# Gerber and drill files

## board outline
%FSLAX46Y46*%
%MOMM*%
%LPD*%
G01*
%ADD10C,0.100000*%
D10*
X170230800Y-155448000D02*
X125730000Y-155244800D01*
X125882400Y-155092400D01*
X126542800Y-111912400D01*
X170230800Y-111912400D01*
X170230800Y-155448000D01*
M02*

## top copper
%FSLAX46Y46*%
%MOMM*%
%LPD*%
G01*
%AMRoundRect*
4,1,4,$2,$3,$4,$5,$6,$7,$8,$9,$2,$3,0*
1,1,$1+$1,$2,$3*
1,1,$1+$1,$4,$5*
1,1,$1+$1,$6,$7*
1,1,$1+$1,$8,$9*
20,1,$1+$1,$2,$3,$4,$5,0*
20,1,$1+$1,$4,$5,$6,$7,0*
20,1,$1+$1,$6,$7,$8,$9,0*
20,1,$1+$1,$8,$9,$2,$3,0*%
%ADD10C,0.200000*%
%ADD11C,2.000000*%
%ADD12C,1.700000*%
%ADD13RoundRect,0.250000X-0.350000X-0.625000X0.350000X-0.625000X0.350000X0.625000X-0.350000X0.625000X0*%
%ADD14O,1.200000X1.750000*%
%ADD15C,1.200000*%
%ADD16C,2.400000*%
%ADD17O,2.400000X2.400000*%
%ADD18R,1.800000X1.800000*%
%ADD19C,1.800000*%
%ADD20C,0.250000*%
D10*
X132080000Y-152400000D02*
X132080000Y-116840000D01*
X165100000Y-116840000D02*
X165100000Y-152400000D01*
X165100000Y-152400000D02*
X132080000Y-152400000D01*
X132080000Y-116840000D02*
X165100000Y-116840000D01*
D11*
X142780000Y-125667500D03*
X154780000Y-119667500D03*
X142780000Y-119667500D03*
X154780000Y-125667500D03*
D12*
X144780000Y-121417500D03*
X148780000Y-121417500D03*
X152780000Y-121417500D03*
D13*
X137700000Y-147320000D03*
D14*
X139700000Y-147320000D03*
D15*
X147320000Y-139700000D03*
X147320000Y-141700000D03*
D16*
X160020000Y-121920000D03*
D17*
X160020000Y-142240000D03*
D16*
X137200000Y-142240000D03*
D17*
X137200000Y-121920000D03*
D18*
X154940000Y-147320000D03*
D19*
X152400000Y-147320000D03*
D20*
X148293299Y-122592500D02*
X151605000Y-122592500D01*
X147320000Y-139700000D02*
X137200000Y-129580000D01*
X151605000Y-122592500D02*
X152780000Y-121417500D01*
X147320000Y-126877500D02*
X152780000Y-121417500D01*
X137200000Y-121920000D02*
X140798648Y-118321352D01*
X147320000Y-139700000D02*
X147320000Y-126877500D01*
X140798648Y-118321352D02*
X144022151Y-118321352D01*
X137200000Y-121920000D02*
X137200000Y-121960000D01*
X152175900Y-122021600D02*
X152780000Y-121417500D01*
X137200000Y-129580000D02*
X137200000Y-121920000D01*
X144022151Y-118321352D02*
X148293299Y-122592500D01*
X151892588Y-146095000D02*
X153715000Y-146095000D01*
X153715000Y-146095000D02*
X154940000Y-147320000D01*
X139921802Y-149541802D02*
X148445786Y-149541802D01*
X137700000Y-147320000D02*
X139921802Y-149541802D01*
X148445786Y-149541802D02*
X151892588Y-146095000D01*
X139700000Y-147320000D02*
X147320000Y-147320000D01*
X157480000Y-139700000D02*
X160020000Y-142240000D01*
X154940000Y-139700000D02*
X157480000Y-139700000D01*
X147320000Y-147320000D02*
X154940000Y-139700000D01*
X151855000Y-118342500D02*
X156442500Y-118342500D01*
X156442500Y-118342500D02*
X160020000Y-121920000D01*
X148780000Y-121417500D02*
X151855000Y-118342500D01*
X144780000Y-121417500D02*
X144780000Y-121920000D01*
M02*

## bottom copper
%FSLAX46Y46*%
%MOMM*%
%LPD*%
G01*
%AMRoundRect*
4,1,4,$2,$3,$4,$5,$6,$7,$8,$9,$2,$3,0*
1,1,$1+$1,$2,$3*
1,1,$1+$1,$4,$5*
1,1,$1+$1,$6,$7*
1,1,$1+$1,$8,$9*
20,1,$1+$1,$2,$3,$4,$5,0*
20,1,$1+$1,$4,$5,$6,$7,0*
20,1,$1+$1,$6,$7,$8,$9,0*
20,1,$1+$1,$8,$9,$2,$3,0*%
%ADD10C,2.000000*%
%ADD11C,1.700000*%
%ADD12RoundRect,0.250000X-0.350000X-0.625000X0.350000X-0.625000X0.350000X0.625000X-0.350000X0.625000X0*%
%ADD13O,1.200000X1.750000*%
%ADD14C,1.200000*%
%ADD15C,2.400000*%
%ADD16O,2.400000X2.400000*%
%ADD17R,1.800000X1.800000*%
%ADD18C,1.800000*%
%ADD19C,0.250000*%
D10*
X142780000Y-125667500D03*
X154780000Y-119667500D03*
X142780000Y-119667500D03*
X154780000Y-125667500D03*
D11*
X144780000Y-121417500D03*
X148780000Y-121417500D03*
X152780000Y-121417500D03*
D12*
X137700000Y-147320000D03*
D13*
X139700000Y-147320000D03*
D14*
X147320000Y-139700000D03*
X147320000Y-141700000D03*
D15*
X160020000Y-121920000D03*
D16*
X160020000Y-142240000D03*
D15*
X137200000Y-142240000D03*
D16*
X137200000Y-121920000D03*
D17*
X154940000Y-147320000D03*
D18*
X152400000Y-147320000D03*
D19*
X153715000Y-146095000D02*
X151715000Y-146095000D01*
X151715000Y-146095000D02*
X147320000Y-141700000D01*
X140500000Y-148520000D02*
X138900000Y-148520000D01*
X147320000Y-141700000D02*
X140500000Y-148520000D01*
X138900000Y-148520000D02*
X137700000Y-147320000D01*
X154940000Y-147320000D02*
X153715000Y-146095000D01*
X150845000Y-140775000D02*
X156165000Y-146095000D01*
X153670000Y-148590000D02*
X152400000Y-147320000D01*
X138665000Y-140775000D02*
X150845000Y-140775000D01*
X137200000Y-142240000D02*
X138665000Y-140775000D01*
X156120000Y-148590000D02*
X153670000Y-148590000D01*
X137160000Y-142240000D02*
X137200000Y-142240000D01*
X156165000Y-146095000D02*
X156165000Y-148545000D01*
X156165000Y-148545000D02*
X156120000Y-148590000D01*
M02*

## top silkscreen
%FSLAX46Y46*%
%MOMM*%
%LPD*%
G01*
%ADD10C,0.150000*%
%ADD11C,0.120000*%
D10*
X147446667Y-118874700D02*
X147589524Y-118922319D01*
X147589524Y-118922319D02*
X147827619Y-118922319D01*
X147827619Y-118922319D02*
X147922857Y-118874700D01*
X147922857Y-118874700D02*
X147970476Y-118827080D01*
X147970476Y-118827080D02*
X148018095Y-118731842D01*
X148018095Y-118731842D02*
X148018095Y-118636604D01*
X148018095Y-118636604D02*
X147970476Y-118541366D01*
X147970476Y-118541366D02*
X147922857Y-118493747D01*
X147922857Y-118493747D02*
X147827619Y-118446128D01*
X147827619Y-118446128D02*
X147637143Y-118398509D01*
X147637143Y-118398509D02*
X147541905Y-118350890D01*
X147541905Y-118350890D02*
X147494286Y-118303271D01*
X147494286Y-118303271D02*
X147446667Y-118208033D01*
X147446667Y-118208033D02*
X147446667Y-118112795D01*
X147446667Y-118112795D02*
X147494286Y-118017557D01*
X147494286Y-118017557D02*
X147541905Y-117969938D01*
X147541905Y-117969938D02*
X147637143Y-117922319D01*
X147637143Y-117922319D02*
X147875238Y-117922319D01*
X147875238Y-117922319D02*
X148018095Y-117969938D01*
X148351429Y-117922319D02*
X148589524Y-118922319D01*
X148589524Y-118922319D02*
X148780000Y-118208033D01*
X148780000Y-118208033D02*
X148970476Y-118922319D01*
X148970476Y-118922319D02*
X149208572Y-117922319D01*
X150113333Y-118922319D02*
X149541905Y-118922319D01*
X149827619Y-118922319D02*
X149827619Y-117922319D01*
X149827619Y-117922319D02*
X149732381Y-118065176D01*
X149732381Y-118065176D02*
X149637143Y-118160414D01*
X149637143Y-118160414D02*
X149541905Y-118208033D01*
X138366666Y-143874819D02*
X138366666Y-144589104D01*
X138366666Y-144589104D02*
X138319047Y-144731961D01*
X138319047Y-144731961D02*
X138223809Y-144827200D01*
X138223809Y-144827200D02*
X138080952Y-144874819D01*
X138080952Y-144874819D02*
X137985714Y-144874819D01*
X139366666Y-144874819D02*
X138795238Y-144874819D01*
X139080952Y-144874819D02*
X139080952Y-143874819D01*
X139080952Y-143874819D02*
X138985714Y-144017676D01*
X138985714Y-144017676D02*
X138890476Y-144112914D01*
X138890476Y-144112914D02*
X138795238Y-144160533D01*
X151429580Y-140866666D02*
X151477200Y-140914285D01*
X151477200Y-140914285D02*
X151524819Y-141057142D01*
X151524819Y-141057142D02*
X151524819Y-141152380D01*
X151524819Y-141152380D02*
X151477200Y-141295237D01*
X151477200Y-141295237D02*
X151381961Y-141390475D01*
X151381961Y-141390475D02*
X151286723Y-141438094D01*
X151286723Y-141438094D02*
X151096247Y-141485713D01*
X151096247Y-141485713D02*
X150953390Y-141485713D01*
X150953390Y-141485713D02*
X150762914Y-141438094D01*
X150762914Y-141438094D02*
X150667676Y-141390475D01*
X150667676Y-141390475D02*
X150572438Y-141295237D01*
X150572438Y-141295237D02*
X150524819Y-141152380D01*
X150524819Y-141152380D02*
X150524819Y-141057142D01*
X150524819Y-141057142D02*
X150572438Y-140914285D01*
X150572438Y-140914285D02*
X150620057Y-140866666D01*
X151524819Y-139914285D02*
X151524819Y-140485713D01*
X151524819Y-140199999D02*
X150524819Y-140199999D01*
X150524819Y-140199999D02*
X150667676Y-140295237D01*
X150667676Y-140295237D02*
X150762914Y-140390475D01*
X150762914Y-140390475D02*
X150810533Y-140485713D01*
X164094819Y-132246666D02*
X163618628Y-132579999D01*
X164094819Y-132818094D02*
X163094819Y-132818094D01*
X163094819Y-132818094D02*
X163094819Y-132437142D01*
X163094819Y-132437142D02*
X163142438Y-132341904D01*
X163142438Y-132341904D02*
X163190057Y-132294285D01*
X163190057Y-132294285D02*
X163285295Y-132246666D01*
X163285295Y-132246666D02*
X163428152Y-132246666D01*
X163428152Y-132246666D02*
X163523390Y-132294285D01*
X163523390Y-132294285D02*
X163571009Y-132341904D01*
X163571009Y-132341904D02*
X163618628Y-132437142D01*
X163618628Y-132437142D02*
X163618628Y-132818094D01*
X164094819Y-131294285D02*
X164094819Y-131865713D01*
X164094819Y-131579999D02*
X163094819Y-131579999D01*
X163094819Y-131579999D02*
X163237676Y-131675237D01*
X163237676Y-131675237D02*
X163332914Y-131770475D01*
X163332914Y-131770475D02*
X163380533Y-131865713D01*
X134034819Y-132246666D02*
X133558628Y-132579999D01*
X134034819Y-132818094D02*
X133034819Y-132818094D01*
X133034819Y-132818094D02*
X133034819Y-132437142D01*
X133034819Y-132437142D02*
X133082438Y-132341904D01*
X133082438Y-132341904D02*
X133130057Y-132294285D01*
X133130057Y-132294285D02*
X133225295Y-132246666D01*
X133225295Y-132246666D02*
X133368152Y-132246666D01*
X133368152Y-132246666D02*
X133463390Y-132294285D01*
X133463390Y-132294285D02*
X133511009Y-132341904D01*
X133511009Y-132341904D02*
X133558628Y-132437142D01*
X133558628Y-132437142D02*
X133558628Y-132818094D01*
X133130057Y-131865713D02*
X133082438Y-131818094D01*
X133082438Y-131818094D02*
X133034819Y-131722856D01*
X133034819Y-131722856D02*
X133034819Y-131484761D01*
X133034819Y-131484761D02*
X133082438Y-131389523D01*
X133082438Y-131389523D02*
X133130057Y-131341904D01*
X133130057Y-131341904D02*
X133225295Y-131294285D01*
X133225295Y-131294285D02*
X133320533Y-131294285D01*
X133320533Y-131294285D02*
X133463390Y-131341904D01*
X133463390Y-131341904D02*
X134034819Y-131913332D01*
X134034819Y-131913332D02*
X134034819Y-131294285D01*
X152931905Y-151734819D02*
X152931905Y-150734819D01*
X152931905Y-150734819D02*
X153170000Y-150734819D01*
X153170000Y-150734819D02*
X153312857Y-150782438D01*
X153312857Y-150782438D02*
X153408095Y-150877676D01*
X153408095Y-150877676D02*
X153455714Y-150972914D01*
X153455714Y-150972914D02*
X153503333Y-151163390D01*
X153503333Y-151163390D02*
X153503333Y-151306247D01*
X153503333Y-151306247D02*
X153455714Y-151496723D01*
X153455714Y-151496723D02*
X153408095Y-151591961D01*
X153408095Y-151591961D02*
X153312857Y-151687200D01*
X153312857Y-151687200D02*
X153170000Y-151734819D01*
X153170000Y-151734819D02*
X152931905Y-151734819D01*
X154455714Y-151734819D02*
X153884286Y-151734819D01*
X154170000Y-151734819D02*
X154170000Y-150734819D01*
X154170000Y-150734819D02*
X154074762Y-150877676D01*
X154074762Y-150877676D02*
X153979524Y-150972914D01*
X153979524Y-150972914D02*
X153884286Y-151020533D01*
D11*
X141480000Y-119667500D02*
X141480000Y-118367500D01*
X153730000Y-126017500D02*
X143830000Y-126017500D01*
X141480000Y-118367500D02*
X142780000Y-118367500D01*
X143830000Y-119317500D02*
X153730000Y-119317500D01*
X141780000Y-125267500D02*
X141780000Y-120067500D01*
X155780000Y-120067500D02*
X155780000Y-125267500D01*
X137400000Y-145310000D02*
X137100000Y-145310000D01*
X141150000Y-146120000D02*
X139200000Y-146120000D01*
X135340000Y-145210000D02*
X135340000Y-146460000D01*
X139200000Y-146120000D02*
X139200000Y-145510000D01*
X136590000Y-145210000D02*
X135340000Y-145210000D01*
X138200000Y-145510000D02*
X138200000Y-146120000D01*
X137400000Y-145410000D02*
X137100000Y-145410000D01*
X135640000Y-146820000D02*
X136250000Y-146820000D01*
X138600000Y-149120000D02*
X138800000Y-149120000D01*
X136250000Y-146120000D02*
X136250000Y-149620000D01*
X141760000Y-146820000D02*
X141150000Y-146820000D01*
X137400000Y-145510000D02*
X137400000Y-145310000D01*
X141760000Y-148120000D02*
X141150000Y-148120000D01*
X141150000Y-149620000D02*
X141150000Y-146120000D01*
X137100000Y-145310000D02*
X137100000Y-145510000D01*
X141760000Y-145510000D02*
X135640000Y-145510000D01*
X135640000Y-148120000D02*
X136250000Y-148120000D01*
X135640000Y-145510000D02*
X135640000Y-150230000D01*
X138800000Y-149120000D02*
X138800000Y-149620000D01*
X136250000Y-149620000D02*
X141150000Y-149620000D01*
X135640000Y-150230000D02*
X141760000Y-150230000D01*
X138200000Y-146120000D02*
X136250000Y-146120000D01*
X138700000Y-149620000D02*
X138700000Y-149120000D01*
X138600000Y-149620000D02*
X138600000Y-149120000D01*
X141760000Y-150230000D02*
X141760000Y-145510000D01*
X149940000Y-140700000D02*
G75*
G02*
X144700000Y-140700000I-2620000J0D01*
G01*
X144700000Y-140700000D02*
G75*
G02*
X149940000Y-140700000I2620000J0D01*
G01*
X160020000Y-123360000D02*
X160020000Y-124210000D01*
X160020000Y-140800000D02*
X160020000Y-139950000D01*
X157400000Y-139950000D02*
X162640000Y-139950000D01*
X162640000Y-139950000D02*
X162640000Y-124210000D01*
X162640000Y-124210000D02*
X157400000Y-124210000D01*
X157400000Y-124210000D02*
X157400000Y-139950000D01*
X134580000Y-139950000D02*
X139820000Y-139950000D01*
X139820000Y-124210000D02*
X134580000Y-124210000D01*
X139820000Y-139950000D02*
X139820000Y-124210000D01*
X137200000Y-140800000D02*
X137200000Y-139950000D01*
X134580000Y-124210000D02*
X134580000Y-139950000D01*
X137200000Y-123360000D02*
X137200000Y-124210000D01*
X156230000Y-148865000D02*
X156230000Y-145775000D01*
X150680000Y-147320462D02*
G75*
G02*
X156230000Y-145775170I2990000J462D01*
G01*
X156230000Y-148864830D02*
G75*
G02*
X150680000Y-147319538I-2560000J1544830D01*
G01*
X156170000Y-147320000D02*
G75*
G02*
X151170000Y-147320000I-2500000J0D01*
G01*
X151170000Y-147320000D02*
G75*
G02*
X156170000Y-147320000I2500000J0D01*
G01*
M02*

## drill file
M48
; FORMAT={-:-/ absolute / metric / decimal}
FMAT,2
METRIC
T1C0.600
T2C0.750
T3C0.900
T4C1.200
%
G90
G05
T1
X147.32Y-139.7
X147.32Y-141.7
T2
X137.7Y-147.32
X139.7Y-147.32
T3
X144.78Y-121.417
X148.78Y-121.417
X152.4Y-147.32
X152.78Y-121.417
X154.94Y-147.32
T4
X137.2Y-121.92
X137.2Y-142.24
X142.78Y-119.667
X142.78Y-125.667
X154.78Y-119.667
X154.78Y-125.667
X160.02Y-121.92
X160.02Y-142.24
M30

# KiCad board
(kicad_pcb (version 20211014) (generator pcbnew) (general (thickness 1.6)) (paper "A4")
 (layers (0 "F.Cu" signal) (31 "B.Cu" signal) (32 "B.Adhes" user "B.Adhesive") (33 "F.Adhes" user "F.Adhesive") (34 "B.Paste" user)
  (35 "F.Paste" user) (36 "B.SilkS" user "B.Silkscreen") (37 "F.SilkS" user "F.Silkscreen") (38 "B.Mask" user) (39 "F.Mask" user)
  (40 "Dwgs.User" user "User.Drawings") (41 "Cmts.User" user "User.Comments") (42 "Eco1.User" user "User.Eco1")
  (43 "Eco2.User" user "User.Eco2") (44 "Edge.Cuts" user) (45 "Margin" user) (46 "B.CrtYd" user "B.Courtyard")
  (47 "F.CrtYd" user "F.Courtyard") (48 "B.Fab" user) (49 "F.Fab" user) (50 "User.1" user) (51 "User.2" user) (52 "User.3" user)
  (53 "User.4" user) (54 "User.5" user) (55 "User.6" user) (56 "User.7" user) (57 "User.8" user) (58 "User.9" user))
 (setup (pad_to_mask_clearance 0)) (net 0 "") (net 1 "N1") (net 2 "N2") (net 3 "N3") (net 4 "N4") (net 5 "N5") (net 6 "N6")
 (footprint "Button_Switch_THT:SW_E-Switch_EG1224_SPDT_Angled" (layer "F.Cu") (at 144.78 121.4175)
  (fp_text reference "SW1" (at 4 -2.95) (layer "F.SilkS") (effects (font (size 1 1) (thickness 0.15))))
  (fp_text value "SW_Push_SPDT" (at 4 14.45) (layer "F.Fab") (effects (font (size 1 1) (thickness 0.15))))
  (fp_line (start -3.3 -1.75) (end -3.3 -3.05) (layer "F.SilkS") (width 0.12))
  (fp_line (start 8.95 4.6) (end -0.95 4.6) (layer "F.SilkS") (width 0.12))
  (fp_line (start -3.3 -3.05) (end -2 -3.05) (layer "F.SilkS") (width 0.12))
  (fp_line (start -0.95 -2.1) (end 8.95 -2.1) (layer "F.SilkS") (width 0.12))
  (fp_line (start -3 3.85) (end -3 -1.35) (layer "F.SilkS") (width 0.12))
  (fp_line (start 11 -1.35) (end 11 3.85) (layer "F.SilkS") (width 0.12))
  (pad "" thru_hole circle (at -2 4.25) (size 2 2) (drill 1.2) (layers *.Cu *.Mask))
  (pad "" thru_hole circle (at 10 -1.75) (size 2 2) (drill 1.2) (layers *.Cu *.Mask))
  (pad "" thru_hole circle (at -2 -1.75) (size 2 2) (drill 1.2) (layers *.Cu *.Mask))
  (pad "" thru_hole circle (at 10 4.25) (size 2 2) (drill 1.2) (layers *.Cu *.Mask))
  (pad "1" thru_hole circle (at 0 0) (size 1.7 1.7) (drill 0.9) (layers *.Cu *.Mask) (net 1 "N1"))
  (pad "2" thru_hole circle (at 4 0) (size 1.7 1.7) (drill 0.9) (layers *.Cu *.Mask) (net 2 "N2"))
  (pad "3" thru_hole circle (at 8 0) (size 1.7 1.7) (drill 0.9) (layers *.Cu *.Mask) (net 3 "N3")))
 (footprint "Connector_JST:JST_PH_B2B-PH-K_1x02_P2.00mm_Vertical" (layer "F.Cu") (at 137.7 147.32)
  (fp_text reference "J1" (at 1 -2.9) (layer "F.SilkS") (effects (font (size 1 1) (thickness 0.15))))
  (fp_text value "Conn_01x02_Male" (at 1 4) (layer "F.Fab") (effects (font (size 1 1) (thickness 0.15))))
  (fp_line (start -0.3 -2.01) (end -0.6 -2.01) (layer "F.SilkS") (width 0.12))
  (fp_line (start 3.45 -1.2) (end 1.5 -1.2) (layer "F.SilkS") (width 0.12))
  (fp_line (start -2.36 -2.11) (end -2.36 -0.86) (layer "F.SilkS") (width 0.12))
  (fp_line (start 1.5 -1.2) (end 1.5 -1.81) (layer "F.SilkS") (width 0.12))
  (fp_line (start -1.11 -2.11) (end -2.36 -2.11) (layer "F.SilkS") (width 0.12))
  (fp_line (start 0.5 -1.81) (end 0.5 -1.2) (layer "F.SilkS") (width 0.12))
  (fp_line (start -0.3 -1.91) (end -0.6 -1.91) (layer "F.SilkS") (width 0.12))
  (fp_line (start -2.06 -0.5) (end -1.45 -0.5) (layer "F.SilkS") (width 0.12))
  (fp_line (start 0.9 1.8) (end 1.1 1.8) (layer "F.SilkS") (width 0.12))
  (fp_line (start -1.45 -1.2) (end -1.45 2.3) (layer "F.SilkS") (width 0.12))
  (fp_line (start 4.06 -0.5) (end 3.45 -0.5) (layer "F.SilkS") (width 0.12))
  (fp_line (start -0.3 -1.81) (end -0.3 -2.01) (layer "F.SilkS") (width 0.12))
  (fp_line (start 4.06 0.8) (end 3.45 0.8) (layer "F.SilkS") (width 0.12))
  (fp_line (start 3.45 2.3) (end 3.45 -1.2) (layer "F.SilkS") (width 0.12))
  (fp_line (start -0.6 -2.01) (end -0.6 -1.81) (layer "F.SilkS") (width 0.12))
  (fp_line (start 4.06 -1.81) (end -2.06 -1.81) (layer "F.SilkS") (width 0.12))
  (fp_line (start -2.06 0.8) (end -1.45 0.8) (layer "F.SilkS") (width 0.12))
  (fp_line (start -2.06 -1.81) (end -2.06 2.91) (layer "F.SilkS") (width 0.12))
  (fp_line (start 1.1 1.8) (end 1.1 2.3) (layer "F.SilkS") (width 0.12))
  (fp_line (start -1.45 2.3) (end 3.45 2.3) (layer "F.SilkS") (width 0.12))
  (fp_line (start -2.06 2.91) (end 4.06 2.91) (layer "F.SilkS") (width 0.12))
  (fp_line (start 0.5 -1.2) (end -1.45 -1.2) (layer "F.SilkS") (width 0.12))
  (fp_line (start 1 2.3) (end 1 1.8) (layer "F.SilkS") (width 0.12))
  (fp_line (start 0.9 2.3) (end 0.9 1.8) (layer "F.SilkS") (width 0.12))
  (fp_line (start 4.06 2.91) (end 4.06 -1.81) (layer "F.SilkS") (width 0.12))
  (pad "1" thru_hole roundrect (at 0 0) (size 1.2 1.75) (drill 0.75) (layers *.Cu *.Mask) (roundrect_rratio 0.208333) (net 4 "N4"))
  (pad "2" thru_hole oval (at 2 0) (size 1.2 1.75) (drill 0.75) (layers *.Cu *.Mask) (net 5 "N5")))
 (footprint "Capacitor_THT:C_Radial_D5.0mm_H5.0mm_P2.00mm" (layer "F.Cu") (at 147.32 139.7 -90)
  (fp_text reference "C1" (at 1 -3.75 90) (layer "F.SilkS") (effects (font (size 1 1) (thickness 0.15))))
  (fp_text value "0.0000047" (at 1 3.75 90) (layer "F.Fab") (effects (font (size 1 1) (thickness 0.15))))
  (fp_circle (center 1 0) (end 3.62 0) (layer "F.SilkS") (width 0.12) (fill none))
  (pad "1" thru_hole circle (at 0 0 270) (size 1.2 1.2) (drill 0.6) (layers *.Cu *.Mask) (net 3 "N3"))
  (pad "2" thru_hole circle (at 2 0 270) (size 1.2 1.2) (drill 0.6) (layers *.Cu *.Mask) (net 4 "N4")))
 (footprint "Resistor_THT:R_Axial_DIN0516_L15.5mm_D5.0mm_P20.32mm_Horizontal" (layer "F.Cu") (at 160.02 121.92 -90)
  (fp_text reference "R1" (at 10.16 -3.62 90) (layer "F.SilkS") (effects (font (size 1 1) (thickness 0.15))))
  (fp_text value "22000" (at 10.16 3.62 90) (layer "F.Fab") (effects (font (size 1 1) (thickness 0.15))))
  (fp_line (start 1.44 0) (end 2.29 0) (layer "F.SilkS") (width 0.12))
  (fp_line (start 18.88 0) (end 18.03 0) (layer "F.SilkS") (width 0.12))
  (fp_line (start 18.03 2.62) (end 18.03 -2.62) (layer "F.SilkS") (width 0.12))
  (fp_line (start 18.03 -2.62) (end 2.29 -2.62) (layer "F.SilkS") (width 0.12))
  (fp_line (start 2.29 -2.62) (end 2.29 2.62) (layer "F.SilkS") (width 0.12))
  (fp_line (start 2.29 2.62) (end 18.03 2.62) (layer "F.SilkS") (width 0.12))
  (pad "1" thru_hole circle (at 0 0 270) (size 2.4 2.4) (drill 1.2) (layers *.Cu *.Mask) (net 2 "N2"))
  (pad "2" thru_hole oval (at 20.32 0 270) (size 2.4 2.4) (drill 1.2) (layers *.Cu *.Mask) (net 5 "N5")))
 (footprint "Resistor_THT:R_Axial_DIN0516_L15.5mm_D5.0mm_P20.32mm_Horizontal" (layer "F.Cu") (at 137.2 142.24 90)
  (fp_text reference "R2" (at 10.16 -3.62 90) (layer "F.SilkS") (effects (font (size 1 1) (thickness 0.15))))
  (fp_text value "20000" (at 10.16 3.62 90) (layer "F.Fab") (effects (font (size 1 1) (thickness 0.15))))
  (fp_line (start 2.29 -2.62) (end 2.29 2.62) (layer "F.SilkS") (width 0.12))
  (fp_line (start 18.03 2.62) (end 18.03 -2.62) (layer "F.SilkS") (width 0.12))
  (fp_line (start 2.29 2.62) (end 18.03 2.62) (layer "F.SilkS") (width 0.12))
  (fp_line (start 1.44 0) (end 2.29 0) (layer "F.SilkS") (width 0.12))
  (fp_line (start 18.03 -2.62) (end 2.29 -2.62) (layer "F.SilkS") (width 0.12))
  (fp_line (start 18.88 0) (end 18.03 0) (layer "F.SilkS") (width 0.12))
  (pad "1" thru_hole circle (at 0 0 90) (size 2.4 2.4) (drill 1.2) (layers *.Cu *.Mask) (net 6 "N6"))
  (pad "2" thru_hole oval (at 20.32 0 90) (size 2.4 2.4) (drill 1.2) (layers *.Cu *.Mask) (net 3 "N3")))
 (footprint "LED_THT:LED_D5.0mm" (layer "F.Cu") (at 154.94 147.32 180)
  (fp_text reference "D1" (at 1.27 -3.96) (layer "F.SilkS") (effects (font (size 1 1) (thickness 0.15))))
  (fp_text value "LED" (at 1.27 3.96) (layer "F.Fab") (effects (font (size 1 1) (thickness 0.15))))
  (fp_line (start -1.29 -1.545) (end -1.29 1.545) (layer "F.SilkS") (width 0.12))
  (fp_arc (start 4.26 -0.000462) (mid 2.072002 2.880433) (end -1.29 1.54483) (layer "F.SilkS") (width 0.12))
  (fp_arc (start -1.29 -1.54483) (mid 2.072002 -2.880433) (end 4.26 0.000462) (layer "F.SilkS") (width 0.12))
  (fp_circle (center 1.27 0) (end 3.77 0) (layer "F.SilkS") (width 0.12) (fill none))
  (pad "1" thru_hole rect (at 0 0 180) (size 1.8 1.8) (drill 0.9) (layers *.Cu *.Mask) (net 4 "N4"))
  (pad "2" thru_hole circle (at 2.54 0 180) (size 1.8 1.8) (drill 0.9) (layers *.Cu *.Mask) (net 6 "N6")))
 (gr_line (start 132.08 152.4) (end 132.08 116.84) (layer "F.Cu") (width 0.2))
 (gr_line (start 165.1 116.84) (end 165.1 152.4) (layer "F.Cu") (width 0.2))
 (gr_line (start 165.1 152.4) (end 132.08 152.4) (layer "F.Cu") (width 0.2))
 (gr_line (start 132.08 116.84) (end 165.1 116.84) (layer "F.Cu") (width 0.2))
 (gr_poly
  (pts (xy 170.2308 155.448) (xy 125.73 155.2448) (xy 125.8824 155.0924) (xy 126.5428 111.9124) (xy 170.2308 111.9124)) (layer "Edge.Cuts")
  (width 0.1) (fill none))
 (segment (start 148.293299 122.5925) (end 151.605 122.5925) (width 0.25) (layer "F.Cu") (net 3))
 (segment (start 147.32 139.7) (end 137.2 129.58) (width 0.25) (layer "F.Cu") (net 3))
 (segment (start 151.605 122.5925) (end 152.78 121.4175) (width 0.25) (layer "F.Cu") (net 3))
 (segment (start 147.32 126.8775) (end 152.78 121.4175) (width 0.25) (layer "F.Cu") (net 3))
 (segment (start 137.2 121.92) (end 140.798648 118.321352) (width 0.25) (layer "F.Cu") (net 3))
 (segment (start 147.32 139.7) (end 147.32 126.8775) (width 0.25) (layer "F.Cu") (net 3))
 (segment (start 140.798648 118.321352) (end 144.022151 118.321352) (width 0.25) (layer "F.Cu") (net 3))
 (segment (start 137.2 121.92) (end 137.2 121.96) (width 0.25) (layer "F.Cu") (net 3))
 (segment (start 152.1759 122.0216) (end 152.78 121.4175) (width 0.25) (layer "F.Cu") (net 3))
 (segment (start 137.2 129.58) (end 137.2 121.92) (width 0.25) (layer "F.Cu") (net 3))
 (segment (start 144.022151 118.321352) (end 148.293299 122.5925) (width 0.25) (layer "F.Cu") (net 3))
 (segment (start 151.892588 146.095) (end 153.715 146.095) (width 0.25) (layer "F.Cu") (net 4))
 (segment (start 153.715 146.095) (end 154.94 147.32) (width 0.25) (layer "F.Cu") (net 4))
 (segment (start 139.921802 149.541802) (end 148.445786 149.541802) (width 0.25) (layer "F.Cu") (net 4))
 (segment (start 137.7 147.32) (end 139.921802 149.541802) (width 0.25) (layer "F.Cu") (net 4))
 (segment (start 148.445786 149.541802) (end 151.892588 146.095) (width 0.25) (layer "F.Cu") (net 4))
 (segment (start 153.715 146.095) (end 151.715 146.095) (width 0.25) (layer "B.Cu") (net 4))
 (segment (start 151.715 146.095) (end 147.32 141.7) (width 0.25) (layer "B.Cu") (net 4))
 (segment (start 140.5 148.52) (end 138.9 148.52) (width 0.25) (layer "B.Cu") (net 4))
 (segment (start 147.32 141.7) (end 140.5 148.52) (width 0.25) (layer "B.Cu") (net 4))
 (segment (start 138.9 148.52) (end 137.7 147.32) (width 0.25) (layer "B.Cu") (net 4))
 (segment (start 154.94 147.32) (end 153.715 146.095) (width 0.25) (layer "B.Cu") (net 4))
 (segment (start 150.845 140.775) (end 156.165 146.095) (width 0.25) (layer "B.Cu") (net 6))
 (segment (start 153.67 148.59) (end 152.4 147.32) (width 0.25) (layer "B.Cu") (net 6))
 (segment (start 138.665 140.775) (end 150.845 140.775) (width 0.25) (layer "B.Cu") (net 6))
 (segment (start 137.2 142.24) (end 138.665 140.775) (width 0.25) (layer "B.Cu") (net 6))
 (segment (start 156.12 148.59) (end 153.67 148.59) (width 0.25) (layer "B.Cu") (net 6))
 (segment (start 137.16 142.24) (end 137.2 142.24) (width 0.25) (layer "B.Cu") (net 6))
 (segment (start 156.165 146.095) (end 156.165 148.545) (width 0.25) (layer "B.Cu") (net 6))
 (segment (start 156.165 148.545) (end 156.12 148.59) (width 0.25) (layer "B.Cu") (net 6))
 (segment (start 139.7 147.32) (end 147.32 147.32) (width 0.25) (layer "F.Cu") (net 5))
 (segment (start 157.48 139.7) (end 160.02 142.24) (width 0.25) (layer "F.Cu") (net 5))
 (segment (start 154.94 139.7) (end 157.48 139.7) (width 0.25) (layer "F.Cu") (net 5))
 (segment (start 147.32 147.32) (end 154.94 139.7) (width 0.25) (layer "F.Cu") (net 5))
 (segment (start 151.855 118.3425) (end 156.4425 118.3425) (width 0.25) (layer "F.Cu") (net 2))
 (segment (start 156.4425 118.3425) (end 160.02 121.92) (width 0.25) (layer "F.Cu") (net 2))
 (segment (start 148.78 121.4175) (end 151.855 118.3425) (width 0.25) (layer "F.Cu") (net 2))
 (segment (start 144.78 121.4175) (end 144.78 121.92) (width 0.25) (layer "F.Cu") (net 1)))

